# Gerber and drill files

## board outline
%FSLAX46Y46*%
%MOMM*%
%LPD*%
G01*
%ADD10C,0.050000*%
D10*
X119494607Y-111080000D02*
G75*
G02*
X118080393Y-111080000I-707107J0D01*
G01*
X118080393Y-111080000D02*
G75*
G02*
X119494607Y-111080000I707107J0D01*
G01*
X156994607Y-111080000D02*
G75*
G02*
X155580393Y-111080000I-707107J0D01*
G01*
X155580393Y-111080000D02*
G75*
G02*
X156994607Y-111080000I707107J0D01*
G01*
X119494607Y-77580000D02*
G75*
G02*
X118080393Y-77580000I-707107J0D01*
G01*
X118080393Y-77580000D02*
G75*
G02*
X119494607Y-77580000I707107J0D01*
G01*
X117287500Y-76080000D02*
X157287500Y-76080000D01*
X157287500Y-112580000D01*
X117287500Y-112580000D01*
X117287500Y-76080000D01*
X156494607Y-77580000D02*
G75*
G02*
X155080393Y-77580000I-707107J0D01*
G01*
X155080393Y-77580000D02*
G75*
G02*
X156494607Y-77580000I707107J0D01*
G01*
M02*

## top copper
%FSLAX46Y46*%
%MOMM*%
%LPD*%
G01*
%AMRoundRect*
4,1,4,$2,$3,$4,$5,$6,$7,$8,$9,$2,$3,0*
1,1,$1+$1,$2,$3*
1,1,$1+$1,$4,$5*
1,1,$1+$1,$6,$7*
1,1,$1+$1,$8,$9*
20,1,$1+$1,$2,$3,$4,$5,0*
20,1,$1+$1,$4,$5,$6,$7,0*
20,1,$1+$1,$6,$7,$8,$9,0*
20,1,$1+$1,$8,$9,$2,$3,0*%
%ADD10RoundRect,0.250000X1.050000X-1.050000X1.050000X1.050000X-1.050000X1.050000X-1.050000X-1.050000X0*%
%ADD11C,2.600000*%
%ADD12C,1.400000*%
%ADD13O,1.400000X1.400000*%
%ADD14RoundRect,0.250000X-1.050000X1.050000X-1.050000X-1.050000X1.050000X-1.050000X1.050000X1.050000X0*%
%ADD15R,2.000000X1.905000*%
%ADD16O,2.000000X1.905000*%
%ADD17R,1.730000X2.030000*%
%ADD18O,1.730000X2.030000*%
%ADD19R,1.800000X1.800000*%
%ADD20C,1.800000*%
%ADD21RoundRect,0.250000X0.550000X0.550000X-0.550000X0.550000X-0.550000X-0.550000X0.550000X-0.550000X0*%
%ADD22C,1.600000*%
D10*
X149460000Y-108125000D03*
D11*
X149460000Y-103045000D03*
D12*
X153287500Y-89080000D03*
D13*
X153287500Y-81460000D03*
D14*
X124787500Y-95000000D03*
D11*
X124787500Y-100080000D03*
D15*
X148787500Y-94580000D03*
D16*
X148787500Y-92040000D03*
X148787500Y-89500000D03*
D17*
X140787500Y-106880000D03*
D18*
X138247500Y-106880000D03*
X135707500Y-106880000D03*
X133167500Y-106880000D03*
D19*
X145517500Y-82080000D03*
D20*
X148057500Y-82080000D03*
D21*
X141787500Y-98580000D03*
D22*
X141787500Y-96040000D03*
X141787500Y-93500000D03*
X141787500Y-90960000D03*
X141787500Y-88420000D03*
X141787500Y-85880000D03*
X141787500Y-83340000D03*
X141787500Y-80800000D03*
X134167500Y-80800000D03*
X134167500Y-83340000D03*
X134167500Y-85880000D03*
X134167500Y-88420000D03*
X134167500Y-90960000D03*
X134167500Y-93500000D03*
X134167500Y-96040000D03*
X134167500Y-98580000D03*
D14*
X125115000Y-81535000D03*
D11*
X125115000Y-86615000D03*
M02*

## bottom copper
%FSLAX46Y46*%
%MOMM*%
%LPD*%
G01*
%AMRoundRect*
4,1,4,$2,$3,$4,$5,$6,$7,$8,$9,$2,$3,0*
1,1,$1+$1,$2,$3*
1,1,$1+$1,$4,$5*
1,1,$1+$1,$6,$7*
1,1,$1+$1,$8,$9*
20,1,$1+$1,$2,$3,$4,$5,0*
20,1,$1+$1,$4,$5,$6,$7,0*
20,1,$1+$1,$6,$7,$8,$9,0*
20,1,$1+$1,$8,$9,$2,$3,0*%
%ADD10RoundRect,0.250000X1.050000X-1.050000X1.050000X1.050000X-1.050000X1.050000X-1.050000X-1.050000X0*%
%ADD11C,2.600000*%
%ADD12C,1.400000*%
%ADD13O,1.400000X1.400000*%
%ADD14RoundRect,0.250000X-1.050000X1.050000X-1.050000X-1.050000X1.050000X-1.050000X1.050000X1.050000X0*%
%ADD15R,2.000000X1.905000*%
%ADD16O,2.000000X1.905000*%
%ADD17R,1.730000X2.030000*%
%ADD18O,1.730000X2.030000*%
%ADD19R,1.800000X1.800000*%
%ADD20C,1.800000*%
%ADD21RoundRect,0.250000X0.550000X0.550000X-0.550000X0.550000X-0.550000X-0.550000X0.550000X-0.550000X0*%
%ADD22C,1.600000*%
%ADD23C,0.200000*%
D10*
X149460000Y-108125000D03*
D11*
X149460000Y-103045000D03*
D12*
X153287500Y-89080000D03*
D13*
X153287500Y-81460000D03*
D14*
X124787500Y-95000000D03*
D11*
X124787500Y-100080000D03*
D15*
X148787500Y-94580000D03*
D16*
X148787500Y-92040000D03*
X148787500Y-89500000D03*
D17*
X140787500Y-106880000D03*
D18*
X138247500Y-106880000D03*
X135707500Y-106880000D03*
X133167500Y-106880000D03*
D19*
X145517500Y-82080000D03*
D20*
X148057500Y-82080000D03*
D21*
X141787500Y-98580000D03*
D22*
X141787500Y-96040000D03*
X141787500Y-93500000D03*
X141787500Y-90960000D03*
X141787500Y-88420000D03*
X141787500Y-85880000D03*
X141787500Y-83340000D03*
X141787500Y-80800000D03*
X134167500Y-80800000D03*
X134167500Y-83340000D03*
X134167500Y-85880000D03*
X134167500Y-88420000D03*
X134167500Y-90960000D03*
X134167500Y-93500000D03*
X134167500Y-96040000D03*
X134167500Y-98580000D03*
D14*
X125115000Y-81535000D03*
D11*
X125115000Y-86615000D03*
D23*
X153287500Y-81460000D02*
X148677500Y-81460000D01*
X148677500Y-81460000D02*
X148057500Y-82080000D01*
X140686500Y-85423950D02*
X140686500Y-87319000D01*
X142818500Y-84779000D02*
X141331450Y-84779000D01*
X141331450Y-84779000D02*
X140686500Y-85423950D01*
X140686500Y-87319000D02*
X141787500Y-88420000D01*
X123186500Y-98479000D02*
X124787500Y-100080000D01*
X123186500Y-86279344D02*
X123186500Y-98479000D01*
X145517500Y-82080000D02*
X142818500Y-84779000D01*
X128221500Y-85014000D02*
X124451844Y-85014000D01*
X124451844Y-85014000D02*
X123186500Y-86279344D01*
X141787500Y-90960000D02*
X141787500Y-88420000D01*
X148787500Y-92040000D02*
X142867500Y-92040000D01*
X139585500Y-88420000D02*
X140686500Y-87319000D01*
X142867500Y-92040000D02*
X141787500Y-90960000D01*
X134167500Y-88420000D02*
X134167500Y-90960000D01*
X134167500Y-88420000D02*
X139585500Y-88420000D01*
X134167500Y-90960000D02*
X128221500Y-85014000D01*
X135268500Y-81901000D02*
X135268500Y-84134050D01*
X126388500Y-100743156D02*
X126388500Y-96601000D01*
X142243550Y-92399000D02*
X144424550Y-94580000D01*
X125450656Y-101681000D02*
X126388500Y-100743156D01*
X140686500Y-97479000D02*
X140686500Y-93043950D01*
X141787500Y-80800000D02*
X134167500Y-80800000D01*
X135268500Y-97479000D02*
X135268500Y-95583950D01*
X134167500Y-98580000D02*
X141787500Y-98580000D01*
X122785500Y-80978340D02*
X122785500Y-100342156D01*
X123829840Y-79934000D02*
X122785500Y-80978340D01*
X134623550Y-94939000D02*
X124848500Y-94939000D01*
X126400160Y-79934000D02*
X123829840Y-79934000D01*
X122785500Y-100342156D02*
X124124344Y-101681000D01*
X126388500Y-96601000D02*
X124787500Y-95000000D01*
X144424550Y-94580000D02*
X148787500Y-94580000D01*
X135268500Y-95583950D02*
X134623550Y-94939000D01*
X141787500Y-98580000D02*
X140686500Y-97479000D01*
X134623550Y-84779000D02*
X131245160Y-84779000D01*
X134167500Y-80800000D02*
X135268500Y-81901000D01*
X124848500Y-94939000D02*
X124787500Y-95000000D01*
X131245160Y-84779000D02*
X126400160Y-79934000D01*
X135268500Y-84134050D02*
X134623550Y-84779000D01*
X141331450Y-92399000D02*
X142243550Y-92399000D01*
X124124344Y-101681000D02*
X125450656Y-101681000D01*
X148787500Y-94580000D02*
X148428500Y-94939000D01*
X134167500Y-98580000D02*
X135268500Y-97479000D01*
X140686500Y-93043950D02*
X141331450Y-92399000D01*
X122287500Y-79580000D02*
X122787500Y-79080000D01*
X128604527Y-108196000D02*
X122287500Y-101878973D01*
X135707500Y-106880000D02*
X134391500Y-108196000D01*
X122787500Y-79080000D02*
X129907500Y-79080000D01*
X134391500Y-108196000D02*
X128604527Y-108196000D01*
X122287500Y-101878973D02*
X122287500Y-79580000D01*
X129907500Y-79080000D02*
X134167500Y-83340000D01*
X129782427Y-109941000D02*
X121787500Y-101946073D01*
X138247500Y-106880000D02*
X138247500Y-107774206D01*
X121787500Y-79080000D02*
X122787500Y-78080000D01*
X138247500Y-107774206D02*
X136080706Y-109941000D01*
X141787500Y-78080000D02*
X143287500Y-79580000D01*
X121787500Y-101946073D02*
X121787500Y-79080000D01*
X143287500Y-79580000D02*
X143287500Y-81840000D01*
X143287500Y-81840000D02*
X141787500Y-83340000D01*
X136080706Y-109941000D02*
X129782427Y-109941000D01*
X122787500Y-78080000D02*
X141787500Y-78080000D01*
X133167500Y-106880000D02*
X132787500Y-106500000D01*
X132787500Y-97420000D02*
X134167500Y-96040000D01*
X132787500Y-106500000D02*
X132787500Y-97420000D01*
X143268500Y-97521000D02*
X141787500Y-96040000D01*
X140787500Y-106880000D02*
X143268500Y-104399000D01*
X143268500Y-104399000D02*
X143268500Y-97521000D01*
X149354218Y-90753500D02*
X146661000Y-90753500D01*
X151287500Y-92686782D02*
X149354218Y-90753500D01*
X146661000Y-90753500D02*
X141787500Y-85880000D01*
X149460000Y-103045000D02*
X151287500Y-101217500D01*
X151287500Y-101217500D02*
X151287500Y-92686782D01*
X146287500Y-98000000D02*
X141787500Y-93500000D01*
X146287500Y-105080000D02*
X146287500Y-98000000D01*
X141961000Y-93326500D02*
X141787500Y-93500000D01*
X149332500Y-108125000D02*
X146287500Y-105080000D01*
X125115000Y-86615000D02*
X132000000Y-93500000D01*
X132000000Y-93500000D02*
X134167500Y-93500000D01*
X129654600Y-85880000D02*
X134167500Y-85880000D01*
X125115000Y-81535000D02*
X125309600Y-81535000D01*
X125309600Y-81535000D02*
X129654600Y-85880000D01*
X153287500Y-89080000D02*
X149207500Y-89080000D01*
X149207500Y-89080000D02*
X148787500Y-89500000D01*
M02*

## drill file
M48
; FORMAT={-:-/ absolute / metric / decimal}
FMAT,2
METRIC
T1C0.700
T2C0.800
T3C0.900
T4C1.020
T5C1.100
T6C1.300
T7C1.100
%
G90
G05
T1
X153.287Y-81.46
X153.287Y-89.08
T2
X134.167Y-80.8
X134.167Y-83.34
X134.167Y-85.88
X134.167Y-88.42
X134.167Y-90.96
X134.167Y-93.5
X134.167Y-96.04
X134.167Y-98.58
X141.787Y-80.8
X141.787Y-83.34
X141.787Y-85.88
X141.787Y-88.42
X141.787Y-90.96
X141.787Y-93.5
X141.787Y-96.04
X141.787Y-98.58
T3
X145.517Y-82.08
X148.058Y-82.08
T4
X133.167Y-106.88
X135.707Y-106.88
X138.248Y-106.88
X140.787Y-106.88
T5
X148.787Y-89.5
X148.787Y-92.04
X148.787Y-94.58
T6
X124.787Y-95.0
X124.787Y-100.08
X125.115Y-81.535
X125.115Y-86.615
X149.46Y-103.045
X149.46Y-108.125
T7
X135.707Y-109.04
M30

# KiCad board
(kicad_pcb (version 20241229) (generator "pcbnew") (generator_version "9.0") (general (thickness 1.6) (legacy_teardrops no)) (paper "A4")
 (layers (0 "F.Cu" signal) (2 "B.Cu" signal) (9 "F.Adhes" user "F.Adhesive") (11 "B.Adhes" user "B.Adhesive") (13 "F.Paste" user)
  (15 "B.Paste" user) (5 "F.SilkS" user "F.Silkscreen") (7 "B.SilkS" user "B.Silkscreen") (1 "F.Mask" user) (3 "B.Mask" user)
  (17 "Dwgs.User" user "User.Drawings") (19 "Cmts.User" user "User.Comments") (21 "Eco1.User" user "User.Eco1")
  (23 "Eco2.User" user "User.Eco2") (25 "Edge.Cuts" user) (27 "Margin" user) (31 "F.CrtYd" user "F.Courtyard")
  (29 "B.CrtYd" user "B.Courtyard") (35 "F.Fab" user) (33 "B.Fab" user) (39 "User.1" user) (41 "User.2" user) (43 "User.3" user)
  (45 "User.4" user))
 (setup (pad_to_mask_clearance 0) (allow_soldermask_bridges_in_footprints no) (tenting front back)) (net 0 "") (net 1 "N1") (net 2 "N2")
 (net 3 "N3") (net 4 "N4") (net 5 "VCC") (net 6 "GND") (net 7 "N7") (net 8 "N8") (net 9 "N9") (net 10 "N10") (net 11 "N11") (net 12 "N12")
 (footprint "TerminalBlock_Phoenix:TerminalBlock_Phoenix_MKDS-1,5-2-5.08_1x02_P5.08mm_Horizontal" (layer "F.Cu") (at 149.46 108.125 90)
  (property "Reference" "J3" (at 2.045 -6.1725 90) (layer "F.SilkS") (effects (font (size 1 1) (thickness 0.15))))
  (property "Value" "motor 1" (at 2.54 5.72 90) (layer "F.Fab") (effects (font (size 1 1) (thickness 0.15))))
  (pad "1" thru_hole roundrect (at 0 0 90) (size 2.6 2.6) (drill 1.3) (layers "*.Cu" "*.Mask") (remove_unused_layers no)
   (roundrect_rratio 0.096154) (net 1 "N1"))
  (pad "2" thru_hole circle (at 5.08 0 90) (size 2.6 2.6) (drill 1.3) (layers "*.Cu" "*.Mask") (remove_unused_layers no) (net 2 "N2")))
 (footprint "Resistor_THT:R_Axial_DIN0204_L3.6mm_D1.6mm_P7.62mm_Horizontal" (layer "F.Cu") (at 153.2875 89.08 90)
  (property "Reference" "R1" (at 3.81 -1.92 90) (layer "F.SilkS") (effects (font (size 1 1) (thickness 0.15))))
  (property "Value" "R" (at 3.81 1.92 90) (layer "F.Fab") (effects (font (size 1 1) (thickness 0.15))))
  (pad "1" thru_hole circle (at 0 0 90) (size 1.4 1.4) (drill 0.7) (layers "*.Cu" "*.Mask") (remove_unused_layers no) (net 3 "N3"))
  (pad "2" thru_hole oval (at 7.62 0 90) (size 1.4 1.4) (drill 0.7) (layers "*.Cu" "*.Mask") (remove_unused_layers no) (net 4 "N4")))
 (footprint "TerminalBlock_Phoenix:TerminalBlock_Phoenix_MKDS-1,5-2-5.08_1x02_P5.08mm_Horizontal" (layer "F.Cu") (at 124.7875 95 -90)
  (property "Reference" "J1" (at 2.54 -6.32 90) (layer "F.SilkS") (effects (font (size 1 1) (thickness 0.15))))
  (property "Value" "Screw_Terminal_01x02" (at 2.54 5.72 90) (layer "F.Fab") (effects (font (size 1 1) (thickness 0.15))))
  (pad "1" thru_hole roundrect (at 0 0 270) (size 2.6 2.6) (drill 1.3) (layers "*.Cu" "*.Mask") (remove_unused_layers no)
   (roundrect_rratio 0.096154) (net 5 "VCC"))
  (pad "2" thru_hole circle (at 5.08 0 270) (size 2.6 2.6) (drill 1.3) (layers "*.Cu" "*.Mask") (remove_unused_layers no) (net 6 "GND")))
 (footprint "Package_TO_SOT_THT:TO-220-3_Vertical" (layer "F.Cu") (at 148.7875 94.58 90)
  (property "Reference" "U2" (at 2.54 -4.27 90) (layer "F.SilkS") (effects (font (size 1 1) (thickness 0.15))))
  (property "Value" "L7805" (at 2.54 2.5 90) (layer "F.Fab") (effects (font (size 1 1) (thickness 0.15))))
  (pad "1" thru_hole rect (at 0 0 90) (size 1.905 2) (drill 1.1) (layers "*.Cu" "*.Mask") (remove_unused_layers no) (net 5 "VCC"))
  (pad "2" thru_hole oval (at 2.54 0 90) (size 1.905 2) (drill 1.1) (layers "*.Cu" "*.Mask") (remove_unused_layers no) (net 6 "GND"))
  (pad "3" thru_hole oval (at 5.08 0 90) (size 1.905 2) (drill 1.1) (layers "*.Cu" "*.Mask") (remove_unused_layers no) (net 3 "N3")))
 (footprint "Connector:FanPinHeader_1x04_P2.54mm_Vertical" (layer "F.Cu") (at 140.7875 106.88 180)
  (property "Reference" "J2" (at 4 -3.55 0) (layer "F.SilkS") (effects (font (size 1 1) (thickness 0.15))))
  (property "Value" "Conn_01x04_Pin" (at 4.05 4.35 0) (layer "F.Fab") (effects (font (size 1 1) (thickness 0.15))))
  (pad "" np_thru_hole circle (at 5.08 -2.16 270) (size 1.1 1.1) (drill 1.1) (layers "*.Cu" "*.Mask"))
  (pad "1" thru_hole rect (at 0 0 270) (size 2.03 1.73) (drill 1.02) (layers "*.Cu" "*.Mask") (remove_unused_layers no) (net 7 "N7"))
  (pad "2" thru_hole oval (at 2.54 0 270) (size 2.03 1.73) (drill 1.02) (layers "*.Cu" "*.Mask") (remove_unused_layers no) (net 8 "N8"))
  (pad "3" thru_hole oval (at 5.08 0 270) (size 2.03 1.73) (drill 1.02) (layers "*.Cu" "*.Mask") (remove_unused_layers no) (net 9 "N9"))
  (pad "4" thru_hole oval (at 7.62 0 270) (size 2.03 1.73) (drill 1.02) (layers "*.Cu" "*.Mask") (remove_unused_layers no) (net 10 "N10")))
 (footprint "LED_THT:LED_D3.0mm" (layer "F.Cu") (at 145.5175 82.08)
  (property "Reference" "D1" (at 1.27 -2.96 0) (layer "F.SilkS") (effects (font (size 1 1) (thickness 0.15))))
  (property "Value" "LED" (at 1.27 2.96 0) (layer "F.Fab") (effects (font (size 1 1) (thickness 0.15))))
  (pad "1" thru_hole rect (at 0 0) (size 1.8 1.8) (drill 0.9) (layers "*.Cu" "*.Mask") (remove_unused_layers no) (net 6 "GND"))
  (pad "2" thru_hole circle (at 2.54 0) (size 1.8 1.8) (drill 0.9) (layers "*.Cu" "*.Mask") (remove_unused_layers no) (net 4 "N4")))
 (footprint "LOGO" (layer "F.Cu") (at 125.2875 107.58)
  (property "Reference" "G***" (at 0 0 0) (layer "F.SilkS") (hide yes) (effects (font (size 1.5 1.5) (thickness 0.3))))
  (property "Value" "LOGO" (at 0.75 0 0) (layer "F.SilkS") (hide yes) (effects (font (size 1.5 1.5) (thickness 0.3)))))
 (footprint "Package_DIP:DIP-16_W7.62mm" (layer "F.Cu") (at 141.7875 98.58 180)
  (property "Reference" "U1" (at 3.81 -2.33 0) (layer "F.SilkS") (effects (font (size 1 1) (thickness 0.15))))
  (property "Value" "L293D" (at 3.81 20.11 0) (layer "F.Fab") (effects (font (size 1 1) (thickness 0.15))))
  (pad "1" thru_hole roundrect (at 0 0 180) (size 1.6 1.6) (drill 0.8) (layers "*.Cu" "*.Mask") (remove_unused_layers no)
   (roundrect_rratio 0.15625) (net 5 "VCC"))
  (pad "2" thru_hole circle (at 0 2.54 180) (size 1.6 1.6) (drill 0.8) (layers "*.Cu" "*.Mask") (remove_unused_layers no) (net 7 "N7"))
  (pad "3" thru_hole circle (at 0 5.08 180) (size 1.6 1.6) (drill 0.8) (layers "*.Cu" "*.Mask") (remove_unused_layers no) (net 1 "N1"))
  (pad "4" thru_hole circle (at 0 7.62 180) (size 1.6 1.6) (drill 0.8) (layers "*.Cu" "*.Mask") (remove_unused_layers no) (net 6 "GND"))
  (pad "5" thru_hole circle (at 0 10.16 180) (size 1.6 1.6) (drill 0.8) (layers "*.Cu" "*.Mask") (remove_unused_layers no) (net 6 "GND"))
  (pad "6" thru_hole circle (at 0 12.7 180) (size 1.6 1.6) (drill 0.8) (layers "*.Cu" "*.Mask") (remove_unused_layers no) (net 2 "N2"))
  (pad "7" thru_hole circle (at 0 15.24 180) (size 1.6 1.6) (drill 0.8) (layers "*.Cu" "*.Mask") (remove_unused_layers no) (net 8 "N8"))
  (pad "8" thru_hole circle (at 0 17.78 180) (size 1.6 1.6) (drill 0.8) (layers "*.Cu" "*.Mask") (remove_unused_layers no) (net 5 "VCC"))
  (pad "9" thru_hole circle (at 7.62 17.78 180) (size 1.6 1.6) (drill 0.8) (layers "*.Cu" "*.Mask") (remove_unused_layers no) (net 5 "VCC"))
  (pad "10" thru_hole circle (at 7.62 15.24 180) (size 1.6 1.6) (drill 0.8) (layers "*.Cu" "*.Mask") (remove_unused_layers no) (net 9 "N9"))
  (pad "11" thru_hole circle (at 7.62 12.7 180) (size 1.6 1.6) (drill 0.8) (layers "*.Cu" "*.Mask") (remove_unused_layers no) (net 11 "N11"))
  (pad "12" thru_hole circle (at 7.62 10.16 180) (size 1.6 1.6) (drill 0.8) (layers "*.Cu" "*.Mask") (remove_unused_layers no) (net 6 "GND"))
  (pad "13" thru_hole circle (at 7.62 7.62 180) (size 1.6 1.6) (drill 0.8) (layers "*.Cu" "*.Mask") (remove_unused_layers no) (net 6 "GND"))
  (pad "14" thru_hole circle (at 7.62 5.08 180) (size 1.6 1.6) (drill 0.8) (layers "*.Cu" "*.Mask") (remove_unused_layers no) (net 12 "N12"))
  (pad "15" thru_hole circle (at 7.62 2.54 180) (size 1.6 1.6) (drill 0.8) (layers "*.Cu" "*.Mask") (remove_unused_layers no) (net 10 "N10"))
  (pad "16" thru_hole circle (at 7.62 0 180) (size 1.6 1.6) (drill 0.8) (layers "*.Cu" "*.Mask") (remove_unused_layers no) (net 5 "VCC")))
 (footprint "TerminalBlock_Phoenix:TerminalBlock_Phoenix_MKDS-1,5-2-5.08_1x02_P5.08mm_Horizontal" (layer "F.Cu") (at 125.115 81.535 -90)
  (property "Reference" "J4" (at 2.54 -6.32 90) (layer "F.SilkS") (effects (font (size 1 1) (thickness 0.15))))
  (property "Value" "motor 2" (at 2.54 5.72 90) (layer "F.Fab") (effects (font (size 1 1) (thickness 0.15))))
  (pad "1" thru_hole roundrect (at 0 0 270) (size 2.6 2.6) (drill 1.3) (layers "*.Cu" "*.Mask") (remove_unused_layers no)
   (roundrect_rratio 0.096154) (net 11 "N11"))
  (pad "2" thru_hole circle (at 5.08 0 270) (size 2.6 2.6) (drill 1.3) (layers "*.Cu" "*.Mask") (remove_unused_layers no) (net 12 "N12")))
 (gr_circle (center 118.7875 111.08) (end 118.2875 111.58) (stroke (width 0.05) (type default)) (fill no) (layer "Edge.Cuts"))
 (gr_circle (center 156.2875 111.08) (end 155.7875 111.58) (stroke (width 0.05) (type default)) (fill no) (layer "Edge.Cuts"))
 (gr_circle (center 118.7875 77.58) (end 118.2875 78.08) (stroke (width 0.05) (type default)) (fill no) (layer "Edge.Cuts"))
 (gr_rect (start 117.2875 76.08) (end 157.2875 112.58) (stroke (width 0.05) (type default)) (fill no) (layer "Edge.Cuts"))
 (gr_circle (center 155.7875 77.58) (end 155.2875 78.08) (stroke (width 0.05) (type default)) (fill no) (layer "Edge.Cuts"))
 (segment (start 153.2875 81.46) (end 148.6775 81.46) (width 0.2) (layer "B.Cu") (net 4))
 (segment (start 148.6775 81.46) (end 148.0575 82.08) (width 0.2) (layer "B.Cu") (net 4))
 (segment (start 140.6865 85.42395) (end 140.6865 87.319) (width 0.2) (layer "B.Cu") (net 6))
 (segment (start 142.8185 84.779) (end 141.33145 84.779) (width 0.2) (layer "B.Cu") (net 6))
 (segment (start 141.33145 84.779) (end 140.6865 85.42395) (width 0.2) (layer "B.Cu") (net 6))
 (segment (start 140.6865 87.319) (end 141.7875 88.42) (width 0.2) (layer "B.Cu") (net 6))
 (segment (start 123.1865 98.479) (end 124.7875 100.08) (width 0.2) (layer "B.Cu") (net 6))
 (segment (start 123.1865 86.279344) (end 123.1865 98.479) (width 0.2) (layer "B.Cu") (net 6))
 (segment (start 145.5175 82.08) (end 142.8185 84.779) (width 0.2) (layer "B.Cu") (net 6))
 (segment (start 128.2215 85.014) (end 124.451844 85.014) (width 0.2) (layer "B.Cu") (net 6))
 (segment (start 124.451844 85.014) (end 123.1865 86.279344) (width 0.2) (layer "B.Cu") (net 6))
 (segment (start 141.7875 90.96) (end 141.7875 88.42) (width 0.2) (layer "B.Cu") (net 6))
 (segment (start 148.7875 92.04) (end 142.8675 92.04) (width 0.2) (layer "B.Cu") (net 6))
 (segment (start 139.5855 88.42) (end 140.6865 87.319) (width 0.2) (layer "B.Cu") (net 6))
 (segment (start 142.8675 92.04) (end 141.7875 90.96) (width 0.2) (layer "B.Cu") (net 6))
 (segment (start 134.1675 88.42) (end 134.1675 90.96) (width 0.2) (layer "B.Cu") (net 6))
 (segment (start 134.1675 88.42) (end 139.5855 88.42) (width 0.2) (layer "B.Cu") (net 6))
 (segment (start 134.1675 90.96) (end 128.2215 85.014) (width 0.2) (layer "B.Cu") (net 6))
 (segment (start 135.2685 81.901) (end 135.2685 84.13405) (width 0.2) (layer "B.Cu") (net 5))
 (segment (start 126.3885 100.743156) (end 126.3885 96.601) (width 0.2) (layer "B.Cu") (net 5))
 (segment (start 142.24355 92.399) (end 144.42455 94.58) (width 0.2) (layer "B.Cu") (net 5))
 (segment (start 125.450656 101.681) (end 126.3885 100.743156) (width 0.2) (layer "B.Cu") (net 5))
 (segment (start 140.6865 97.479) (end 140.6865 93.04395) (width 0.2) (layer "B.Cu") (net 5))
 (segment (start 141.7875 80.8) (end 134.1675 80.8) (width 0.2) (layer "B.Cu") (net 5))
 (segment (start 135.2685 97.479) (end 135.2685 95.58395) (width 0.2) (layer "B.Cu") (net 5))
 (segment (start 134.1675 98.58) (end 141.7875 98.58) (width 0.2) (layer "B.Cu") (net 5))
 (segment (start 122.7855 80.97834) (end 122.7855 100.342156) (width 0.2) (layer "B.Cu") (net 5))
 (segment (start 123.82984 79.934) (end 122.7855 80.97834) (width 0.2) (layer "B.Cu") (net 5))
 (segment (start 134.62355 94.939) (end 124.8485 94.939) (width 0.2) (layer "B.Cu") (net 5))
 (segment (start 126.40016 79.934) (end 123.82984 79.934) (width 0.2) (layer "B.Cu") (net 5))
 (segment (start 122.7855 100.342156) (end 124.124344 101.681) (width 0.2) (layer "B.Cu") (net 5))
 (segment (start 126.3885 96.601) (end 124.7875 95) (width 0.2) (layer "B.Cu") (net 5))
 (segment (start 144.42455 94.58) (end 148.7875 94.58) (width 0.2) (layer "B.Cu") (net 5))
 (segment (start 135.2685 95.58395) (end 134.62355 94.939) (width 0.2) (layer "B.Cu") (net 5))
 (segment (start 141.7875 98.58) (end 140.6865 97.479) (width 0.2) (layer "B.Cu") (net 5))
 (segment (start 134.62355 84.779) (end 131.24516 84.779) (width 0.2) (layer "B.Cu") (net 5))
 (segment (start 134.1675 80.8) (end 135.2685 81.901) (width 0.2) (layer "B.Cu") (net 5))
 (segment (start 124.8485 94.939) (end 124.7875 95) (width 0.2) (layer "B.Cu") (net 5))
 (segment (start 131.24516 84.779) (end 126.40016 79.934) (width 0.2) (layer "B.Cu") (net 5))
 (segment (start 135.2685 84.13405) (end 134.62355 84.779) (width 0.2) (layer "B.Cu") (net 5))
 (segment (start 141.33145 92.399) (end 142.24355 92.399) (width 0.2) (layer "B.Cu") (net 5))
 (segment (start 124.124344 101.681) (end 125.450656 101.681) (width 0.2) (layer "B.Cu") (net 5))
 (segment (start 148.7875 94.58) (end 148.4285 94.939) (width 0.2) (layer "B.Cu") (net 5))
 (segment (start 134.1675 98.58) (end 135.2685 97.479) (width 0.2) (layer "B.Cu") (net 5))
 (segment (start 140.6865 93.04395) (end 141.33145 92.399) (width 0.2) (layer "B.Cu") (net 5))
 (segment (start 122.2875 79.58) (end 122.7875 79.08) (width 0.2) (layer "B.Cu") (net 9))
 (segment (start 128.604527 108.196) (end 122.2875 101.878973) (width 0.2) (layer "B.Cu") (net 9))
 (segment (start 135.7075 106.88) (end 134.3915 108.196) (width 0.2) (layer "B.Cu") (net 9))
 (segment (start 122.7875 79.08) (end 129.9075 79.08) (width 0.2) (layer "B.Cu") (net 9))
 (segment (start 134.3915 108.196) (end 128.604527 108.196) (width 0.2) (layer "B.Cu") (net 9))
 (segment (start 122.2875 101.878973) (end 122.2875 79.58) (width 0.2) (layer "B.Cu") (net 9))
 (segment (start 129.9075 79.08) (end 134.1675 83.34) (width 0.2) (layer "B.Cu") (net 9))
 (segment (start 129.782427 109.941) (end 121.7875 101.946073) (width 0.2) (layer "B.Cu") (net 8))
 (segment (start 138.2475 106.88) (end 138.2475 107.774206) (width 0.2) (layer "B.Cu") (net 8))
 (segment (start 121.7875 79.08) (end 122.7875 78.08) (width 0.2) (layer "B.Cu") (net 8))
 (segment (start 138.2475 107.774206) (end 136.080706 109.941) (width 0.2) (layer "B.Cu") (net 8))
 (segment (start 141.7875 78.08) (end 143.2875 79.58) (width 0.2) (layer "B.Cu") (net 8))
 (segment (start 121.7875 101.946073) (end 121.7875 79.08) (width 0.2) (layer "B.Cu") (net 8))
 (segment (start 143.2875 79.58) (end 143.2875 81.84) (width 0.2) (layer "B.Cu") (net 8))
 (segment (start 143.2875 81.84) (end 141.7875 83.34) (width 0.2) (layer "B.Cu") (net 8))
 (segment (start 136.080706 109.941) (end 129.782427 109.941) (width 0.2) (layer "B.Cu") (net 8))
 (segment (start 122.7875 78.08) (end 141.7875 78.08) (width 0.2) (layer "B.Cu") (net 8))
 (segment (start 133.1675 106.88) (end 132.7875 106.5) (width 0.2) (layer "B.Cu") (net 10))
 (segment (start 132.7875 97.42) (end 134.1675 96.04) (width 0.2) (layer "B.Cu") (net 10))
 (segment (start 132.7875 106.5) (end 132.7875 97.42) (width 0.2) (layer "B.Cu") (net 10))
 (segment (start 143.2685 97.521) (end 141.7875 96.04) (width 0.2) (layer "B.Cu") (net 7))
 (segment (start 140.7875 106.88) (end 143.2685 104.399) (width 0.2) (layer "B.Cu") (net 7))
 (segment (start 143.2685 104.399) (end 143.2685 97.521) (width 0.2) (layer "B.Cu") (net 7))
 (segment (start 149.354218 90.7535) (end 146.661 90.7535) (width 0.2) (layer "B.Cu") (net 2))
 (segment (start 151.2875 92.686782) (end 149.354218 90.7535) (width 0.2) (layer "B.Cu") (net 2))
 (segment (start 146.661 90.7535) (end 141.7875 85.88) (width 0.2) (layer "B.Cu") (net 2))
 (segment (start 149.46 103.045) (end 151.2875 101.2175) (width 0.2) (layer "B.Cu") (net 2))
 (segment (start 151.2875 101.2175) (end 151.2875 92.686782) (width 0.2) (layer "B.Cu") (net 2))
 (segment (start 146.2875 98) (end 141.7875 93.5) (width 0.2) (layer "B.Cu") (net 1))
 (segment (start 146.2875 105.08) (end 146.2875 98) (width 0.2) (layer "B.Cu") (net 1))
 (segment (start 141.961 93.3265) (end 141.7875 93.5) (width 0.2) (layer "B.Cu") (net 1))
 (segment (start 149.3325 108.125) (end 146.2875 105.08) (width 0.2) (layer "B.Cu") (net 1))
 (segment (start 125.115 86.615) (end 132 93.5) (width 0.2) (layer "B.Cu") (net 12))
 (segment (start 132 93.5) (end 134.1675 93.5) (width 0.2) (layer "B.Cu") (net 12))
 (segment (start 129.6546 85.88) (end 134.1675 85.88) (width 0.2) (layer "B.Cu") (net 11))
 (segment (start 125.115 81.535) (end 125.3096 81.535) (width 0.2) (layer "B.Cu") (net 11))
 (segment (start 125.3096 81.535) (end 129.6546 85.88) (width 0.2) (layer "B.Cu") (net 11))
 (segment (start 153.2875 89.08) (end 149.2075 89.08) (width 0.2) (layer "B.Cu") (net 3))
 (segment (start 149.2075 89.08) (end 148.7875 89.5) (width 0.2) (layer "B.Cu") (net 3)))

